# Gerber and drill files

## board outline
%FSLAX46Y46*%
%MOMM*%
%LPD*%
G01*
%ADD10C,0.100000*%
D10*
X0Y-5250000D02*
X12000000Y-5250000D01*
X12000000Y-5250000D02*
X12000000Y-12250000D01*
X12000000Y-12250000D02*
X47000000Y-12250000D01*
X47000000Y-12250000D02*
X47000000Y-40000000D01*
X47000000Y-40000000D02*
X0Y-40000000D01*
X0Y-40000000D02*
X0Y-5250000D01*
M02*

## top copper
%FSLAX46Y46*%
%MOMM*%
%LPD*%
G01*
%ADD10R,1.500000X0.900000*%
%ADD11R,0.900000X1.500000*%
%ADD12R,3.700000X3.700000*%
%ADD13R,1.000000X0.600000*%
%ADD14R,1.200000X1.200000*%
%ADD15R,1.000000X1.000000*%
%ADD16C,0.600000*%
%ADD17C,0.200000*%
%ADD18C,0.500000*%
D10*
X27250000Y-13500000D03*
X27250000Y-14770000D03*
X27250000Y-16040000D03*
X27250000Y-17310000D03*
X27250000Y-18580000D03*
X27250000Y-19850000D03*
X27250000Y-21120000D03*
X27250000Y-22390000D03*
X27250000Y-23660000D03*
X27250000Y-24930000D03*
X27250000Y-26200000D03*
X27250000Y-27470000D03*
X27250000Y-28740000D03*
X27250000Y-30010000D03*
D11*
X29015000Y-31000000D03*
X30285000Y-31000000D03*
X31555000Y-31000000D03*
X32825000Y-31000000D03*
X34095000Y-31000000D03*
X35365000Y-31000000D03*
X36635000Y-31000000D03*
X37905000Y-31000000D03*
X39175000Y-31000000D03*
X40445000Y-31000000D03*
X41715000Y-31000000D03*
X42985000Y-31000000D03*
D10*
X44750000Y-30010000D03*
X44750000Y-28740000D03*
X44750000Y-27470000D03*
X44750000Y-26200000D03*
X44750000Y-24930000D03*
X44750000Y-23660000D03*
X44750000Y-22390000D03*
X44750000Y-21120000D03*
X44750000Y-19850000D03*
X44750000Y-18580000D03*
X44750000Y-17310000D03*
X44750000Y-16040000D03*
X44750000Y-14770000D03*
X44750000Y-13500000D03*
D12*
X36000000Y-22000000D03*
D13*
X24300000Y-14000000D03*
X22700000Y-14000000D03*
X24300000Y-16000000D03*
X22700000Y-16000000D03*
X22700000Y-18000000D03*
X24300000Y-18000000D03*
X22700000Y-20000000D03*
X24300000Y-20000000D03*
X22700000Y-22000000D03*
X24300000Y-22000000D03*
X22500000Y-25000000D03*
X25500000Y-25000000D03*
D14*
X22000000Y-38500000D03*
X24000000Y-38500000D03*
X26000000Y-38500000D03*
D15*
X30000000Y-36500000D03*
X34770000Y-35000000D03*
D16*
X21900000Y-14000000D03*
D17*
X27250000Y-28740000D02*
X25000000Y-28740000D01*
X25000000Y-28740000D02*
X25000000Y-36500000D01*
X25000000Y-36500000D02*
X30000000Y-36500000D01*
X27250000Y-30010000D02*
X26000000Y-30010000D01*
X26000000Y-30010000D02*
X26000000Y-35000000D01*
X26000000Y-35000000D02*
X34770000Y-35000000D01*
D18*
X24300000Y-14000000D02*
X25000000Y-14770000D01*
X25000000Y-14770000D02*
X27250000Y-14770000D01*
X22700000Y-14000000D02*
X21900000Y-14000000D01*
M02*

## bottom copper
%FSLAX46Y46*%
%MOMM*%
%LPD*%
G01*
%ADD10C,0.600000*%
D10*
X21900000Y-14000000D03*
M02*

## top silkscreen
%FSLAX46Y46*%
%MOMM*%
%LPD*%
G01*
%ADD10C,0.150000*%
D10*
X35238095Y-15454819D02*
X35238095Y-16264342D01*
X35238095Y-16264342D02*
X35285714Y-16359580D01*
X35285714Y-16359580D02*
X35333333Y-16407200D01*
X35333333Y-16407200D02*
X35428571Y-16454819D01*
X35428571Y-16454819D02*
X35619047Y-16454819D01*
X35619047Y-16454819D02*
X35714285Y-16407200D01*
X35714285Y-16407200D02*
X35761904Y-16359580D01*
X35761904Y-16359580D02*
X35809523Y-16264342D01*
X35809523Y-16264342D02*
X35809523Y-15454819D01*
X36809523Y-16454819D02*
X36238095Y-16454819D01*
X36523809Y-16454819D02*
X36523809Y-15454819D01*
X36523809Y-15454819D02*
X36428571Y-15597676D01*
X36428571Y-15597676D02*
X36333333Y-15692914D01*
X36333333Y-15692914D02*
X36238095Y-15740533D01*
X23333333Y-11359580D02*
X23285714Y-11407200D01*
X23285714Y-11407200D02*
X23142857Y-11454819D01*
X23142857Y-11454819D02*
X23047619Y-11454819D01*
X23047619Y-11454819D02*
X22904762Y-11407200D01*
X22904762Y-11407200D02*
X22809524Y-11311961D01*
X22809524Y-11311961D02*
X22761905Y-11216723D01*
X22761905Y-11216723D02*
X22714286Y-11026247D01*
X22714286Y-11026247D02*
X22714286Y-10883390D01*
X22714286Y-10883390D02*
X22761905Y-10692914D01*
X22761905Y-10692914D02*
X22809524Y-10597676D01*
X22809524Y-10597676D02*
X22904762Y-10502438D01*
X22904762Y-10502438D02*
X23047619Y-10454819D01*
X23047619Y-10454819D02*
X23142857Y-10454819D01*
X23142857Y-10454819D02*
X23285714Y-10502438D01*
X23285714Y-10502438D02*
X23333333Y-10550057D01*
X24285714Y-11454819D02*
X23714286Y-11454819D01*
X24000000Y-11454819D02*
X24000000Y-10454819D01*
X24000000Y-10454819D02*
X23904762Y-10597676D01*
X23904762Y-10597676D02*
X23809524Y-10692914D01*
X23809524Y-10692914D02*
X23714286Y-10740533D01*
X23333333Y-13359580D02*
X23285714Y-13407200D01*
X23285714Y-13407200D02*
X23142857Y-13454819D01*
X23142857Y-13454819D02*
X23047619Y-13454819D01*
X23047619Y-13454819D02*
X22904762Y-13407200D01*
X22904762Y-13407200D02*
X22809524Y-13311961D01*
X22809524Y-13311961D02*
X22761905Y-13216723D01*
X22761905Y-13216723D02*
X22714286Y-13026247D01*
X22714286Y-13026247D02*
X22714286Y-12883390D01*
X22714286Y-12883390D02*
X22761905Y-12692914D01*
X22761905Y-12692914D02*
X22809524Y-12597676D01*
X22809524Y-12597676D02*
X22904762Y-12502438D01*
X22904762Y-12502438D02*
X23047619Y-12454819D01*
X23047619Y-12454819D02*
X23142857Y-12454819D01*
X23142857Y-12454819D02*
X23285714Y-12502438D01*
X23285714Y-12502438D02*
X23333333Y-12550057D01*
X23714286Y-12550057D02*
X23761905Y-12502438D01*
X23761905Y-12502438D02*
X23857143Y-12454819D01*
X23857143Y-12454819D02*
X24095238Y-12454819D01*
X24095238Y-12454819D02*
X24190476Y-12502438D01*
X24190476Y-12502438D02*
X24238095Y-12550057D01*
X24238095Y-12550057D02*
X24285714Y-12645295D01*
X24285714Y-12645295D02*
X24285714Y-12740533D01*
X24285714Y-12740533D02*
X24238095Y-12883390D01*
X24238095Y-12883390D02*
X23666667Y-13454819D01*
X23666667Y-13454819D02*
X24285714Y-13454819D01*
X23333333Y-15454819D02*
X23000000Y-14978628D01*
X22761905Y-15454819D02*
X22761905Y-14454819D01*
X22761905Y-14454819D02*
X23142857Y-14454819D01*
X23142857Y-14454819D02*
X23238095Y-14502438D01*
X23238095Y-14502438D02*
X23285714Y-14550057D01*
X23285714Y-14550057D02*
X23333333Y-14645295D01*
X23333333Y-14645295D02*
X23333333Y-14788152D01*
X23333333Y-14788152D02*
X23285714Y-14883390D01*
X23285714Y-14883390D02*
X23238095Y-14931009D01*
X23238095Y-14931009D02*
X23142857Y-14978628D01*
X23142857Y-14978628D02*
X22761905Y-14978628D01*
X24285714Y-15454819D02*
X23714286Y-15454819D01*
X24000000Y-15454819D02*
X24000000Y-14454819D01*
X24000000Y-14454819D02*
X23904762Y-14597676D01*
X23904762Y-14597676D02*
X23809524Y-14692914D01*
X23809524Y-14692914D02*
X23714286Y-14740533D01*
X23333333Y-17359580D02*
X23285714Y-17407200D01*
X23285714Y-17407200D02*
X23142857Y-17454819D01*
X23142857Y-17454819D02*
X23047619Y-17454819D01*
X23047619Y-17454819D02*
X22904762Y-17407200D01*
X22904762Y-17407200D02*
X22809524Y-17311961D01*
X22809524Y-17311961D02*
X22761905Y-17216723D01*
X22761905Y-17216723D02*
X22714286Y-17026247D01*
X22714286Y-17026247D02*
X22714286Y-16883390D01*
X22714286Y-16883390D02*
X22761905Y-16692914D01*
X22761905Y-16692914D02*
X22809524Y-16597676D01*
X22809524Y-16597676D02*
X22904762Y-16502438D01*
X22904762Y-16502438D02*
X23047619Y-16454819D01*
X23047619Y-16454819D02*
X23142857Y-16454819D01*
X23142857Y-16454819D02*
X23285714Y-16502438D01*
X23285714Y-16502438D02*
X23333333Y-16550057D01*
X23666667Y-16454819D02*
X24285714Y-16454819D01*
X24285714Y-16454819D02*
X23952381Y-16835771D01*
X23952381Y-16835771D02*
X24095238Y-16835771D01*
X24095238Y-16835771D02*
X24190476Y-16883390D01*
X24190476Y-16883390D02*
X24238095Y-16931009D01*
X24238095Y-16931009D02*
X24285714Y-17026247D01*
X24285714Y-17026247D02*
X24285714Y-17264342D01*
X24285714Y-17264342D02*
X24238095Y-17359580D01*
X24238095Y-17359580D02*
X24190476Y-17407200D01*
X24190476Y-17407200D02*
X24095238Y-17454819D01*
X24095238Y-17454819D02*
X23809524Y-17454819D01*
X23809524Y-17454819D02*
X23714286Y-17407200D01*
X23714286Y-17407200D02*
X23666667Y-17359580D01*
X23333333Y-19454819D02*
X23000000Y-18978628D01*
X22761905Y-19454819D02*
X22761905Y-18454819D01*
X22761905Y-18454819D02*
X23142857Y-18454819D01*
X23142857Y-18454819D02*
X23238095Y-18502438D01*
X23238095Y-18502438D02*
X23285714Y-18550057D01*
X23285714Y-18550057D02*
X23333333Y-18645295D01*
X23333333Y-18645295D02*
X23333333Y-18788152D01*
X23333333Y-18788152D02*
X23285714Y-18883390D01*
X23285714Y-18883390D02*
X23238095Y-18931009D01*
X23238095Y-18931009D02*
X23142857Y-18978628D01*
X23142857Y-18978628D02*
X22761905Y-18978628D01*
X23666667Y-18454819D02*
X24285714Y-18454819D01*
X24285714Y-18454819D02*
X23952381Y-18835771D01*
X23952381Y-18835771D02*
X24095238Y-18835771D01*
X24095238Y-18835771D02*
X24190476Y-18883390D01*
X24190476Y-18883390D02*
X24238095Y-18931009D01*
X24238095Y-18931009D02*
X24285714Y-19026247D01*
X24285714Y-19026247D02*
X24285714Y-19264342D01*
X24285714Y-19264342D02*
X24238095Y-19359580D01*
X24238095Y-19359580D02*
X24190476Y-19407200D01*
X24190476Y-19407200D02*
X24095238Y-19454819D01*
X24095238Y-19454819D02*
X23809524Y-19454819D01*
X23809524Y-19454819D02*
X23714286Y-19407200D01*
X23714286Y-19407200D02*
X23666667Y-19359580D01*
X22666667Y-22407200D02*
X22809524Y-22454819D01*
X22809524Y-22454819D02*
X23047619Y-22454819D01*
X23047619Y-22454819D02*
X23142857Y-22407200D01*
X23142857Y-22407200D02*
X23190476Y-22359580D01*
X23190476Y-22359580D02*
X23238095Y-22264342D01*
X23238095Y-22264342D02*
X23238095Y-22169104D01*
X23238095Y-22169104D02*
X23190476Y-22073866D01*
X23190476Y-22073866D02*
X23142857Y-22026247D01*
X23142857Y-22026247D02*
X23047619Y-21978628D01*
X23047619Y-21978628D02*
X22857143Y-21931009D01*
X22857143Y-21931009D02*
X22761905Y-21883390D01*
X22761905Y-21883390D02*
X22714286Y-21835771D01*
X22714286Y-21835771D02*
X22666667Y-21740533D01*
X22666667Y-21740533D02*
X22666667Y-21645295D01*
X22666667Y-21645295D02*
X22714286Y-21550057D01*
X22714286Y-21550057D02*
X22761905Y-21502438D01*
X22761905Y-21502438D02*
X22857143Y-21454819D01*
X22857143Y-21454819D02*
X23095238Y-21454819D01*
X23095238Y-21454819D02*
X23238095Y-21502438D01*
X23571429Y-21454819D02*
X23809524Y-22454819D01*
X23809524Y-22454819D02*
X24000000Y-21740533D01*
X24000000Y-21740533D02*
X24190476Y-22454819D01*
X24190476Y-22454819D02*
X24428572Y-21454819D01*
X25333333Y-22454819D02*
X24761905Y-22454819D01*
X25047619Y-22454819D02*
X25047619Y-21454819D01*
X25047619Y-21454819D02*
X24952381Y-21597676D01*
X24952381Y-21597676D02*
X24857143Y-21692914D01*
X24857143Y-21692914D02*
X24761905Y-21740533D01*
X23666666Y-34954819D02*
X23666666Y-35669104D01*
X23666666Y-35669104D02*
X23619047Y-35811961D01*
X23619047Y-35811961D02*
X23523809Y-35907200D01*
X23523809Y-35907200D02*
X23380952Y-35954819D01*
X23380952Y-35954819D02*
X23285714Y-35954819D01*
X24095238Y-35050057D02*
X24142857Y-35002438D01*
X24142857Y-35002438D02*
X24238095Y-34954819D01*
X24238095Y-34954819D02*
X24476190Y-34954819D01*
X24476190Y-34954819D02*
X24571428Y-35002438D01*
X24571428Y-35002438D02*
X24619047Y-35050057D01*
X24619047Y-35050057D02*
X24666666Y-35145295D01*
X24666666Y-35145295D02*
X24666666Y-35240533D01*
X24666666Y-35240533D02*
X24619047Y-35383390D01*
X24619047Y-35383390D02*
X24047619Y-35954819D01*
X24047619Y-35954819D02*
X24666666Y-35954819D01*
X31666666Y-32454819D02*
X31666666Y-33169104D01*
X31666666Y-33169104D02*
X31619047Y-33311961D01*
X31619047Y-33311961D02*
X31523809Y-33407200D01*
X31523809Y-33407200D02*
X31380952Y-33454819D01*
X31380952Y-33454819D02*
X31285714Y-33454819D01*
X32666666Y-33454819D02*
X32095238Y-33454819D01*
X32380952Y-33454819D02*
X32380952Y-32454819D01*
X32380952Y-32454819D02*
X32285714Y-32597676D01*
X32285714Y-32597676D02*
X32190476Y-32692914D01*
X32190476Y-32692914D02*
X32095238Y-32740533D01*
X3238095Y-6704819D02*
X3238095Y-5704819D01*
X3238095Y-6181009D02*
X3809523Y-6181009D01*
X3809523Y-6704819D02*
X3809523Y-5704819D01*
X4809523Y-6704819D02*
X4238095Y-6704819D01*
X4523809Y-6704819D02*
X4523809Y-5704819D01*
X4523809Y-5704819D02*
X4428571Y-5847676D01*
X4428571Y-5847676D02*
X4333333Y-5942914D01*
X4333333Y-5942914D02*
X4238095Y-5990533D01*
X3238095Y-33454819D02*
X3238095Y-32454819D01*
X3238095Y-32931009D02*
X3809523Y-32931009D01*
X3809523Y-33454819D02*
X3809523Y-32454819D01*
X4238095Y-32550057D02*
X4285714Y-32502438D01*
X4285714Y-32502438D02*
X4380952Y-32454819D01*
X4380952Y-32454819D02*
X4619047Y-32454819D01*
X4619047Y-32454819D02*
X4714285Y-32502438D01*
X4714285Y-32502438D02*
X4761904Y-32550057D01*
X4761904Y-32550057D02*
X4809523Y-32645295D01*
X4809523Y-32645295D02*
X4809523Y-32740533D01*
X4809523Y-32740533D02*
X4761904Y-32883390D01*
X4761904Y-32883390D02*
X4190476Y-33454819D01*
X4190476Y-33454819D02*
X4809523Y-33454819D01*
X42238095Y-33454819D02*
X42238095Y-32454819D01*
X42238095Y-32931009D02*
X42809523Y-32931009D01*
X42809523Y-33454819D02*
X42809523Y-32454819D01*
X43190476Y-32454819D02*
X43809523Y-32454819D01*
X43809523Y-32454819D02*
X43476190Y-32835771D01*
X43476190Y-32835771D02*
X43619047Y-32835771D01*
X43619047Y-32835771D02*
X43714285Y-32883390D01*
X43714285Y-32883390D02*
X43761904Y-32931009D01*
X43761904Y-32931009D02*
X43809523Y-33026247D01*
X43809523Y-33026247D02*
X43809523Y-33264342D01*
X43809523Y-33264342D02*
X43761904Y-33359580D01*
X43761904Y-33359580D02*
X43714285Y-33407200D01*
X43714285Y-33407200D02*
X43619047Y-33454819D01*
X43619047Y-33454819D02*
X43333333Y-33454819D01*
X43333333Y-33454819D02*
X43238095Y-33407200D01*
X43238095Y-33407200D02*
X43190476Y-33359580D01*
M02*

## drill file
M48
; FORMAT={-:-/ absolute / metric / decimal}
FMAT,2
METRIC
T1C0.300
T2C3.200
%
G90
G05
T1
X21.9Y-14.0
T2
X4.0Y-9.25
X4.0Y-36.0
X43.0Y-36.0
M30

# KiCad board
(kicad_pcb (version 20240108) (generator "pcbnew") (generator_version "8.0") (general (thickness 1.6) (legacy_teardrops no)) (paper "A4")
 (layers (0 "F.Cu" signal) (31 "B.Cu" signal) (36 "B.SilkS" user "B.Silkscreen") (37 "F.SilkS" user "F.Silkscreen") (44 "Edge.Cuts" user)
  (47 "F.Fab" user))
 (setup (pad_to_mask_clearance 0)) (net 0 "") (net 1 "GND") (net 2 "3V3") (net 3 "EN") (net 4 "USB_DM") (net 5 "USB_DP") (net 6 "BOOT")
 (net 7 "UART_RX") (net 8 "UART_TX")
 (gr_line (start 0 5.25) (end 12 5.25) (stroke (width 0.1) (type default)) (layer "Edge.Cuts"))
 (gr_line (start 12 5.25) (end 12 12.25) (stroke (width 0.1) (type default)) (layer "Edge.Cuts"))
 (gr_line (start 12 12.25) (end 47 12.25) (stroke (width 0.1) (type default)) (layer "Edge.Cuts"))
 (gr_line (start 47 12.25) (end 47 40) (stroke (width 0.1) (type default)) (layer "Edge.Cuts"))
 (gr_line (start 47 40) (end 0 40) (stroke (width 0.1) (type default)) (layer "Edge.Cuts"))
 (gr_line (start 0 40) (end 0 5.25) (stroke (width 0.1) (type default)) (layer "Edge.Cuts"))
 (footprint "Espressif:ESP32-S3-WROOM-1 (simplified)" (layer "F.Cu") (at 36.0 19.0 0)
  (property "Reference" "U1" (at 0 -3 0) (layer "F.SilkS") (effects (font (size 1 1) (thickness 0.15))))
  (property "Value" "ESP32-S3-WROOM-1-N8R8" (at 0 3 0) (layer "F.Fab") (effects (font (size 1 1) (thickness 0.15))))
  (pad "1" smd rect (at -8.750 -5.500 0) (size 1.5 0.9) (layers "F.Cu" "F.Paste" "F.Mask") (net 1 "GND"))
  (pad "2" smd rect (at -8.750 -4.230 0) (size 1.5 0.9) (layers "F.Cu" "F.Paste" "F.Mask") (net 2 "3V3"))
  (pad "3" smd rect (at -8.750 -2.960 0) (size 1.5 0.9) (layers "F.Cu" "F.Paste" "F.Mask") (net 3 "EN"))
  (pad "4" smd rect (at -8.750 -1.690 0) (size 1.5 0.9) (layers "F.Cu" "F.Paste" "F.Mask"))
  (pad "5" smd rect (at -8.750 -0.420 0) (size 1.5 0.9) (layers "F.Cu" "F.Paste" "F.Mask"))
  (pad "6" smd rect (at -8.750 0.850 0) (size 1.5 0.9) (layers "F.Cu" "F.Paste" "F.Mask"))
  (pad "7" smd rect (at -8.750 2.120 0) (size 1.5 0.9) (layers "F.Cu" "F.Paste" "F.Mask"))
  (pad "8" smd rect (at -8.750 3.390 0) (size 1.5 0.9) (layers "F.Cu" "F.Paste" "F.Mask"))
  (pad "9" smd rect (at -8.750 4.660 0) (size 1.5 0.9) (layers "F.Cu" "F.Paste" "F.Mask"))
  (pad "10" smd rect (at -8.750 5.930 0) (size 1.5 0.9) (layers "F.Cu" "F.Paste" "F.Mask"))
  (pad "11" smd rect (at -8.750 7.200 0) (size 1.5 0.9) (layers "F.Cu" "F.Paste" "F.Mask"))
  (pad "12" smd rect (at -8.750 8.470 0) (size 1.5 0.9) (layers "F.Cu" "F.Paste" "F.Mask"))
  (pad "13" smd rect (at -8.750 9.740 0) (size 1.5 0.9) (layers "F.Cu" "F.Paste" "F.Mask") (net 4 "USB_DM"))
  (pad "14" smd rect (at -8.750 11.010 0) (size 1.5 0.9) (layers "F.Cu" "F.Paste" "F.Mask") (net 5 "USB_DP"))
  (pad "15" smd rect (at -6.985 12.000 0) (size 0.9 1.5) (layers "F.Cu" "F.Paste" "F.Mask"))
  (pad "16" smd rect (at -5.715 12.000 0) (size 0.9 1.5) (layers "F.Cu" "F.Paste" "F.Mask"))
  (pad "17" smd rect (at -4.445 12.000 0) (size 0.9 1.5) (layers "F.Cu" "F.Paste" "F.Mask"))
  (pad "18" smd rect (at -3.175 12.000 0) (size 0.9 1.5) (layers "F.Cu" "F.Paste" "F.Mask"))
  (pad "19" smd rect (at -1.905 12.000 0) (size 0.9 1.5) (layers "F.Cu" "F.Paste" "F.Mask"))
  (pad "20" smd rect (at -0.635 12.000 0) (size 0.9 1.5) (layers "F.Cu" "F.Paste" "F.Mask"))
  (pad "21" smd rect (at 0.635 12.000 0) (size 0.9 1.5) (layers "F.Cu" "F.Paste" "F.Mask"))
  (pad "22" smd rect (at 1.905 12.000 0) (size 0.9 1.5) (layers "F.Cu" "F.Paste" "F.Mask"))
  (pad "23" smd rect (at 3.175 12.000 0) (size 0.9 1.5) (layers "F.Cu" "F.Paste" "F.Mask"))
  (pad "24" smd rect (at 4.445 12.000 0) (size 0.9 1.5) (layers "F.Cu" "F.Paste" "F.Mask"))
  (pad "25" smd rect (at 5.715 12.000 0) (size 0.9 1.5) (layers "F.Cu" "F.Paste" "F.Mask"))
  (pad "26" smd rect (at 6.985 12.000 0) (size 0.9 1.5) (layers "F.Cu" "F.Paste" "F.Mask"))
  (pad "27" smd rect (at 8.750 11.010 0) (size 1.5 0.9) (layers "F.Cu" "F.Paste" "F.Mask") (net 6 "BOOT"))
  (pad "28" smd rect (at 8.750 9.740 0) (size 1.5 0.9) (layers "F.Cu" "F.Paste" "F.Mask"))
  (pad "29" smd rect (at 8.750 8.470 0) (size 1.5 0.9) (layers "F.Cu" "F.Paste" "F.Mask"))
  (pad "30" smd rect (at 8.750 7.200 0) (size 1.5 0.9) (layers "F.Cu" "F.Paste" "F.Mask"))
  (pad "31" smd rect (at 8.750 5.930 0) (size 1.5 0.9) (layers "F.Cu" "F.Paste" "F.Mask"))
  (pad "32" smd rect (at 8.750 4.660 0) (size 1.5 0.9) (layers "F.Cu" "F.Paste" "F.Mask"))
  (pad "33" smd rect (at 8.750 3.390 0) (size 1.5 0.9) (layers "F.Cu" "F.Paste" "F.Mask"))
  (pad "34" smd rect (at 8.750 2.120 0) (size 1.5 0.9) (layers "F.Cu" "F.Paste" "F.Mask"))
  (pad "35" smd rect (at 8.750 0.850 0) (size 1.5 0.9) (layers "F.Cu" "F.Paste" "F.Mask"))
  (pad "36" smd rect (at 8.750 -0.420 0) (size 1.5 0.9) (layers "F.Cu" "F.Paste" "F.Mask") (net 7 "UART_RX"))
  (pad "37" smd rect (at 8.750 -1.690 0) (size 1.5 0.9) (layers "F.Cu" "F.Paste" "F.Mask") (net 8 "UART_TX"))
  (pad "38" smd rect (at 8.750 -2.960 0) (size 1.5 0.9) (layers "F.Cu" "F.Paste" "F.Mask"))
  (pad "39" smd rect (at 8.750 -4.230 0) (size 1.5 0.9) (layers "F.Cu" "F.Paste" "F.Mask"))
  (pad "40" smd rect (at 8.750 -5.500 0) (size 1.5 0.9) (layers "F.Cu" "F.Paste" "F.Mask") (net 1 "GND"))
  (pad "41" smd rect (at 0.000 3.000 0) (size 3.7 3.7) (layers "F.Cu" "F.Paste" "F.Mask") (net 1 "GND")))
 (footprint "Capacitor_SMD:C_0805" (layer "F.Cu") (at 23.5 14.0 0)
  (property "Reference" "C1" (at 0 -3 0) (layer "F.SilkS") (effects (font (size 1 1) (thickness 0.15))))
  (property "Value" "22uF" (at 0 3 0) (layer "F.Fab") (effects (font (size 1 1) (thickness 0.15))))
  (pad "1" smd rect (at 0.800 0.000 0) (size 1.0 0.6) (layers "F.Cu" "F.Paste" "F.Mask") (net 2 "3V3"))
  (pad "2" smd rect (at -0.800 0.000 0) (size 1.0 0.6) (layers "F.Cu" "F.Paste" "F.Mask") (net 1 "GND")))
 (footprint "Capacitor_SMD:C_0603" (layer "F.Cu") (at 23.5 16.0 0)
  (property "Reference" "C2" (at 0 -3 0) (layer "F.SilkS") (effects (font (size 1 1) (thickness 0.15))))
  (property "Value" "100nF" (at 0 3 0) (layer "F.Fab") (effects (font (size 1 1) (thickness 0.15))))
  (pad "1" smd rect (at 0.800 0.000 0) (size 1.0 0.6) (layers "F.Cu" "F.Paste" "F.Mask") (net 2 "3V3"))
  (pad "2" smd rect (at -0.800 0.000 0) (size 1.0 0.6) (layers "F.Cu" "F.Paste" "F.Mask") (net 1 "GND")))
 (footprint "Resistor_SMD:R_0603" (layer "F.Cu") (at 23.5 18.0 0)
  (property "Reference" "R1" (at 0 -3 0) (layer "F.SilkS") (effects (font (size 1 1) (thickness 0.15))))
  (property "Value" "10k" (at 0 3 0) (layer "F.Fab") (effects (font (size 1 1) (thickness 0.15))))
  (pad "1" smd rect (at -0.800 0.000 0) (size 1.0 0.6) (layers "F.Cu" "F.Paste" "F.Mask") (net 2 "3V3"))
  (pad "2" smd rect (at 0.800 0.000 0) (size 1.0 0.6) (layers "F.Cu" "F.Paste" "F.Mask") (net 3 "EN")))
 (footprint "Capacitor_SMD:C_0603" (layer "F.Cu") (at 23.5 20.0 0)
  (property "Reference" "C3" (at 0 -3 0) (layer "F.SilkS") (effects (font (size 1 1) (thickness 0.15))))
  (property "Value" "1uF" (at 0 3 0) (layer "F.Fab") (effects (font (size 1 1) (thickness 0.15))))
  (pad "1" smd rect (at -0.800 0.000 0) (size 1.0 0.6) (layers "F.Cu" "F.Paste" "F.Mask") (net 3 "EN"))
  (pad "2" smd rect (at 0.800 0.000 0) (size 1.0 0.6) (layers "F.Cu" "F.Paste" "F.Mask") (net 1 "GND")))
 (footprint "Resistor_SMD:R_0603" (layer "F.Cu") (at 23.5 22.0 0)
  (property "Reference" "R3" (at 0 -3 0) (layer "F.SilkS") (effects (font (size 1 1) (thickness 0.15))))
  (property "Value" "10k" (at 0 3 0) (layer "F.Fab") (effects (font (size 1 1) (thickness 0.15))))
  (pad "1" smd rect (at -0.800 0.000 0) (size 1.0 0.6) (layers "F.Cu" "F.Paste" "F.Mask") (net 2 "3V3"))
  (pad "2" smd rect (at 0.800 0.000 0) (size 1.0 0.6) (layers "F.Cu" "F.Paste" "F.Mask") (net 6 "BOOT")))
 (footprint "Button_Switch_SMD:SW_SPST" (layer "F.Cu") (at 24.0 25.0 0)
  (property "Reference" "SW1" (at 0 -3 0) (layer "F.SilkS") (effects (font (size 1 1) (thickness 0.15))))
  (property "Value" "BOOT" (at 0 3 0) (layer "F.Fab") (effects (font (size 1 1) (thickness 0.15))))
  (pad "1" smd rect (at -1.500 0.000 0) (size 1.0 0.6) (layers "F.Cu" "F.Paste" "F.Mask") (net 6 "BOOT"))
  (pad "2" smd rect (at 1.500 0.000 0) (size 1.0 0.6) (layers "F.Cu" "F.Paste" "F.Mask") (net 1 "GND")))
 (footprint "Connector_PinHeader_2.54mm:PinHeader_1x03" (layer "F.Cu") (at 24.0 38.5 0)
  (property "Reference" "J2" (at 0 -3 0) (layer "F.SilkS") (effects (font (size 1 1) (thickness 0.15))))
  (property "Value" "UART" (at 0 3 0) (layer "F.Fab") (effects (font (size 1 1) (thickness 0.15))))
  (pad "1" smd rect (at -2.000 0.000 0) (size 1.2 1.2) (layers "F.Cu" "F.Paste" "F.Mask") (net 8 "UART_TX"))
  (pad "2" smd rect (at 0.000 0.000 0) (size 1.2 1.2) (layers "F.Cu" "F.Paste" "F.Mask") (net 7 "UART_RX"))
  (pad "3" smd rect (at 2.000 0.000 0) (size 1.2 1.2) (layers "F.Cu" "F.Paste" "F.Mask") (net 1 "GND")))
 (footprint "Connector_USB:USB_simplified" (layer "F.Cu") (at 32.0 36.0 0)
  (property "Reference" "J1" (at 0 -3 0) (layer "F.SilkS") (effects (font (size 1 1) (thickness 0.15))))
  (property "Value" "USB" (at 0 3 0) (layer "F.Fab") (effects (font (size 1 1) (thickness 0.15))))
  (pad "1" smd rect (at -2.000 0.500 0) (size 1.0 1.0) (layers "F.Cu" "F.Paste" "F.Mask") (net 4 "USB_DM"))
  (pad "2" smd rect (at 2.770 -1.000 0) (size 1.0 1.0) (layers "F.Cu" "F.Paste" "F.Mask") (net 5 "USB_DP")))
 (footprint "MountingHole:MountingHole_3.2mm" (layer "F.Cu") (at 4 9.25)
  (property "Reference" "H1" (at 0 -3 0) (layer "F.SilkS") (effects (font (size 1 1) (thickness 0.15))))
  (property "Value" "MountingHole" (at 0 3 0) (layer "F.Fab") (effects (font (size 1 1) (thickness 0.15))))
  (pad "" np_thru_hole circle (at 0 0) (size 3.2 3.2) (drill 3.2) (layers "*.Cu" "*.Mask")))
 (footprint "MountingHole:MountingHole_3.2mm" (layer "F.Cu") (at 4 36)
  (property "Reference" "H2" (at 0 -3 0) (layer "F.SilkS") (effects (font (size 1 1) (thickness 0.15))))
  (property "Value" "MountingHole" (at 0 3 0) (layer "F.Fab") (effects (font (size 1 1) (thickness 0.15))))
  (pad "" np_thru_hole circle (at 0 0) (size 3.2 3.2) (drill 3.2) (layers "*.Cu" "*.Mask")))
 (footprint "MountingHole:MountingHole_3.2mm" (layer "F.Cu") (at 43 36)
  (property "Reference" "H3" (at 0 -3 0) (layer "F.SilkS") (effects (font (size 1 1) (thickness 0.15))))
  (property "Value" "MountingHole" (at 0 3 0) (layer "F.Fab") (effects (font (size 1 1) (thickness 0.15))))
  (pad "" np_thru_hole circle (at 0 0) (size 3.2 3.2) (drill 3.2) (layers "*.Cu" "*.Mask")))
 (segment (start 27.250 28.740) (end 25.000 28.740) (width 0.2) (layer "F.Cu") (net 4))
 (segment (start 25.000 28.740) (end 25.000 36.500) (width 0.2) (layer "F.Cu") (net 4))
 (segment (start 25.000 36.500) (end 30.000 36.500) (width 0.2) (layer "F.Cu") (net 4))
 (segment (start 27.250 30.010) (end 26.000 30.010) (width 0.2) (layer "F.Cu") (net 5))
 (segment (start 26.000 30.010) (end 26.000 35.000) (width 0.2) (layer "F.Cu") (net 5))
 (segment (start 26.000 35.000) (end 34.770 35.000) (width 0.2) (layer "F.Cu") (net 5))
 (segment (start 24.300 14.000) (end 25.000 14.770) (width 0.5) (layer "F.Cu") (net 2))
 (segment (start 25.000 14.770) (end 27.250 14.770) (width 0.5) (layer "F.Cu") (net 2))
 (segment (start 22.700 14.000) (end 21.900 14.000) (width 0.5) (layer "F.Cu") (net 1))
 (via (at 21.9 14.0) (size 0.6) (drill 0.3) (layers "F.Cu" "B.Cu") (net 1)))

